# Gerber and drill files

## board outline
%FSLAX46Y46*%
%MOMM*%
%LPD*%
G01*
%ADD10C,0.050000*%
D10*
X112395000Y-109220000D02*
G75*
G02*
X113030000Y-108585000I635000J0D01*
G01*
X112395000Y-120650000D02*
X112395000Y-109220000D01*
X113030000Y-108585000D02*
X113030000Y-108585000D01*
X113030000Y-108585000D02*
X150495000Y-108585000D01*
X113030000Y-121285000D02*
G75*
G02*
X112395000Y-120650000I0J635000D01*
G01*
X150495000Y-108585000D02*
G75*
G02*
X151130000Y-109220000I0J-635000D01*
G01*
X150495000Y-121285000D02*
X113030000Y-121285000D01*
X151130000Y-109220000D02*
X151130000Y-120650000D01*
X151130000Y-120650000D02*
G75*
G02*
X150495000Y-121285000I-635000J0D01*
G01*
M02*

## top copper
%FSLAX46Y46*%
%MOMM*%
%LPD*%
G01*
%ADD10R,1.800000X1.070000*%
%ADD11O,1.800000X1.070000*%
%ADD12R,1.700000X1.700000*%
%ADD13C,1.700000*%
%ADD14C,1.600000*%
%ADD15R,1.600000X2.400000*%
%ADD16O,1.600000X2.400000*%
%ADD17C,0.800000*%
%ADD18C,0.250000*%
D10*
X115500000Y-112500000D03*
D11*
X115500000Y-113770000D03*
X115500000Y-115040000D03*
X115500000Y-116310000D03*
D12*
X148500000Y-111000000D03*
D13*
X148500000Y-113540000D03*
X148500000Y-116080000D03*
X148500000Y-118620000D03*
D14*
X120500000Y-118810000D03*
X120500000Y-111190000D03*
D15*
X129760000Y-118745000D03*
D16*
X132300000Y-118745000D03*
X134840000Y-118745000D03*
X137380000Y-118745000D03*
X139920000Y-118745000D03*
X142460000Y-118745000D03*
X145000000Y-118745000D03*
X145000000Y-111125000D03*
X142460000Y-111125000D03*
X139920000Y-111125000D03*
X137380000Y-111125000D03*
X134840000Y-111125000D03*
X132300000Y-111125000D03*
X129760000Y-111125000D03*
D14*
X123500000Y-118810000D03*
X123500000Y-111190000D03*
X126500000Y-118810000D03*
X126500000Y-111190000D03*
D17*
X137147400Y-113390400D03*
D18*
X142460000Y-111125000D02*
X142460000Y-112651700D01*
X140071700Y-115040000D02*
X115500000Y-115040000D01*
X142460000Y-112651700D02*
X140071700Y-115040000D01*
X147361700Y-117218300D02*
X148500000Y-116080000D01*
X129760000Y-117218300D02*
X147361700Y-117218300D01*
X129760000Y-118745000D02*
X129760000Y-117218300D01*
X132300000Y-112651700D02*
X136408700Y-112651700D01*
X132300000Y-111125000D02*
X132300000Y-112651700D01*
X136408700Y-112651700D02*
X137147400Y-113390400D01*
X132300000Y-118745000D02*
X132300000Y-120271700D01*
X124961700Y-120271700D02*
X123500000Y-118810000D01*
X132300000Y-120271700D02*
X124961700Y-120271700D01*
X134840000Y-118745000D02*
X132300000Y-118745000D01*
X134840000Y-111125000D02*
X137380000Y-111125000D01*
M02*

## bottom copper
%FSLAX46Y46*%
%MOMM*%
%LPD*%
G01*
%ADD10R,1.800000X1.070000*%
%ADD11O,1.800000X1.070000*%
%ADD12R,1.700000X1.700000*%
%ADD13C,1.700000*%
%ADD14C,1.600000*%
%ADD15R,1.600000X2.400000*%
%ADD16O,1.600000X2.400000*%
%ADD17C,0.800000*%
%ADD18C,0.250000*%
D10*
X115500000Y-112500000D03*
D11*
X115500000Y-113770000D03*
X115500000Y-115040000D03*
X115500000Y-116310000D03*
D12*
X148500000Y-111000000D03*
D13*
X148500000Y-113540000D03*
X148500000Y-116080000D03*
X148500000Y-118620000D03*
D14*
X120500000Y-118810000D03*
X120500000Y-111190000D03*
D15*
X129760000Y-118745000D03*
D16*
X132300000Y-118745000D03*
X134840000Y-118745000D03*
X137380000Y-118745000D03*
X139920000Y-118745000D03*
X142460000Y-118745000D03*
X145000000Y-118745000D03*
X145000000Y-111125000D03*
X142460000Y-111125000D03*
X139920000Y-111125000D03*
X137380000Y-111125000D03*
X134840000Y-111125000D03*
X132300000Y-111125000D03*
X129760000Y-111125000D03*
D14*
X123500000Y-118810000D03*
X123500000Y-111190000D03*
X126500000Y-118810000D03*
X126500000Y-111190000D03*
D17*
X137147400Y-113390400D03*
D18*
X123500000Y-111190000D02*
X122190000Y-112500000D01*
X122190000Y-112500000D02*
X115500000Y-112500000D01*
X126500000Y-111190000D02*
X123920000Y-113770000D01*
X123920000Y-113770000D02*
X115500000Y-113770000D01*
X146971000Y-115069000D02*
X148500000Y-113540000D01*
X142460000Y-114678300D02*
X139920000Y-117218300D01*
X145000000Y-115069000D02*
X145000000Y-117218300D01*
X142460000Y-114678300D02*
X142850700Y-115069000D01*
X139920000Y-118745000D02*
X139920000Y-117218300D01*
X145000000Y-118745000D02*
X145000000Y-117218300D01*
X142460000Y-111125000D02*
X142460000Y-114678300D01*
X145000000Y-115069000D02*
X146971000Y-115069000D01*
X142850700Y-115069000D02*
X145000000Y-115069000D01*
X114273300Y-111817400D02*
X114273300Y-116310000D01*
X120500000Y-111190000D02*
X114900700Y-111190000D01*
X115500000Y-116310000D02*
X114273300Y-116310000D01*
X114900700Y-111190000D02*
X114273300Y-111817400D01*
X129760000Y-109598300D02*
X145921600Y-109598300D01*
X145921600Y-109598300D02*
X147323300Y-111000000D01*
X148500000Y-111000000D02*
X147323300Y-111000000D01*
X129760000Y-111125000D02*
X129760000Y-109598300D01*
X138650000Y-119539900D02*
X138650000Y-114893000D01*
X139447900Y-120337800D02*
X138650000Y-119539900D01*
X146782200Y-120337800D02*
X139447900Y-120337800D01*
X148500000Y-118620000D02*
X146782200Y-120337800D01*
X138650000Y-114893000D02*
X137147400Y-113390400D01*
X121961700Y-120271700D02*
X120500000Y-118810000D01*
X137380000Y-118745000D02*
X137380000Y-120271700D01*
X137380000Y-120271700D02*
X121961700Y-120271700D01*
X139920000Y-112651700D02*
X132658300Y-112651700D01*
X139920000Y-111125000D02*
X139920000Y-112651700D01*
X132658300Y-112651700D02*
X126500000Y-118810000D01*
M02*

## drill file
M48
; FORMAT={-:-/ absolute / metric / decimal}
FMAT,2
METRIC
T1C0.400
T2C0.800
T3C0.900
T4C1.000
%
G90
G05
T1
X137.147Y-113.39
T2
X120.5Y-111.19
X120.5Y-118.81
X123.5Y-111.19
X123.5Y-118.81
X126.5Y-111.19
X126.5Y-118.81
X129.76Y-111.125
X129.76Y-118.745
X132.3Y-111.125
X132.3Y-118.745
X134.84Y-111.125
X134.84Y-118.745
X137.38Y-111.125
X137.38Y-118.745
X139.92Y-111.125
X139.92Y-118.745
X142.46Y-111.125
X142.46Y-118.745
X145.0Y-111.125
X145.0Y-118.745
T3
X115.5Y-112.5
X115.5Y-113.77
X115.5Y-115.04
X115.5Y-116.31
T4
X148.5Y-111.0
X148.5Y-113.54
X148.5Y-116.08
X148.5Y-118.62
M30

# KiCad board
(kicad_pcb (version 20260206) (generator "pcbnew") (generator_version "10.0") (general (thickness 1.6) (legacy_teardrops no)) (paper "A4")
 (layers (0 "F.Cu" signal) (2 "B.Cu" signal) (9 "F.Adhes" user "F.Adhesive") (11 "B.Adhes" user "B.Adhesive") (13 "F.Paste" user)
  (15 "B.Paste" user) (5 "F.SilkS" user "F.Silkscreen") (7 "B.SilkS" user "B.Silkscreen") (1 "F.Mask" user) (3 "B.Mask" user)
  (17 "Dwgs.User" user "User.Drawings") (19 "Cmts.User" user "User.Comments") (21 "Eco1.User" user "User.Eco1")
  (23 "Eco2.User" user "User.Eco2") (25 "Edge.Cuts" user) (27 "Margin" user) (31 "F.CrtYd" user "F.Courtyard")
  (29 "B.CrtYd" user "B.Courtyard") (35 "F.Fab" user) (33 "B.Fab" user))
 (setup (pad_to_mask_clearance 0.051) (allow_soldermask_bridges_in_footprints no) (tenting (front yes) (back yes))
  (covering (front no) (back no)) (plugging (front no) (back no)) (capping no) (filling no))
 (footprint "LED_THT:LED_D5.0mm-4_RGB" (layer "F.Cu") (at 115.5 112.5 -90)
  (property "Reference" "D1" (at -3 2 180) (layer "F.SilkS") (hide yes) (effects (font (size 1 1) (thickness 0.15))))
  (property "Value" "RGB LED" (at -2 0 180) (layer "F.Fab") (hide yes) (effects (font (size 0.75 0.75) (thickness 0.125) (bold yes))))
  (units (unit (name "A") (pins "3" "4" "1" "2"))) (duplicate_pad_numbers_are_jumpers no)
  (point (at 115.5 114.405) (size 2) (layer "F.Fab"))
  (pad "1" thru_hole rect (at 0 0 270) (size 1.07 1.8) (drill 0.9) (layers "*.Cu" "*.Mask") (remove_unused_layers no) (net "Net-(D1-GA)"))
  (pad "2" thru_hole oval (at 1.27 0 270) (size 1.07 1.8) (drill 0.9) (layers "*.Cu" "*.Mask") (remove_unused_layers no) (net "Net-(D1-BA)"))
  (pad "3" thru_hole oval (at 2.54 0 270) (size 1.07 1.8) (drill 0.9) (layers "*.Cu" "*.Mask") (remove_unused_layers no) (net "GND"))
  (pad "4" thru_hole oval (at 3.81 0 270) (size 1.07 1.8) (drill 0.9) (layers "*.Cu" "*.Mask") (remove_unused_layers no) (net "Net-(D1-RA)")))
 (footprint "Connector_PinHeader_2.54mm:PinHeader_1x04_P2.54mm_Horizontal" (layer "F.Cu") (at 148.5 111)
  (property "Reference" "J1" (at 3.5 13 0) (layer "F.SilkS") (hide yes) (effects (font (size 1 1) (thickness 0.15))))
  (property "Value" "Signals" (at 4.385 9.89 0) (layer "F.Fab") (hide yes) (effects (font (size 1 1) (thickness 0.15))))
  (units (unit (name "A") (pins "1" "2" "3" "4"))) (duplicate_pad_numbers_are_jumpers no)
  (pad "1" thru_hole rect (at 0 0) (size 1.7 1.7) (drill 1) (layers "*.Cu" "*.Mask") (remove_unused_layers no) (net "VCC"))
  (pad "2" thru_hole circle (at 0 2.54) (size 1.7 1.7) (drill 1) (layers "*.Cu" "*.Mask") (remove_unused_layers no) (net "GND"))
  (pad "3" thru_hole circle (at 0 5.08) (size 1.7 1.7) (drill 1) (layers "*.Cu" "*.Mask") (remove_unused_layers no) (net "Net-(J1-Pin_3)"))
  (pad "4" thru_hole circle (at 0 7.62) (size 1.7 1.7) (drill 1) (layers "*.Cu" "*.Mask") (remove_unused_layers no) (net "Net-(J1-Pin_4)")))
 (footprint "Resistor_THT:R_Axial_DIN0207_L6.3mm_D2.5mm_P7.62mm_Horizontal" (layer "F.Cu") (at 120.5 118.81 90)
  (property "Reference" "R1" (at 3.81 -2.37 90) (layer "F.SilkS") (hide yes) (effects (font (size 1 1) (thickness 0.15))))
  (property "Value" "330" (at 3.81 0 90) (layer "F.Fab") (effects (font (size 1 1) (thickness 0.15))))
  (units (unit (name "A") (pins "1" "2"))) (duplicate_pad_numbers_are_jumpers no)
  (pad "1" thru_hole circle (at 0 0 90) (size 1.6 1.6) (drill 0.8) (layers "*.Cu" "*.Mask") (remove_unused_layers no) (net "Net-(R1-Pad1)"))
  (pad "2" thru_hole circle (at 7.62 0 90) (size 1.6 1.6) (drill 0.8) (layers "*.Cu" "*.Mask") (remove_unused_layers no) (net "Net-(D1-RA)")))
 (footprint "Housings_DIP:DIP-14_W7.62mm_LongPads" (layer "F.Cu") (at 129.76 118.745 90)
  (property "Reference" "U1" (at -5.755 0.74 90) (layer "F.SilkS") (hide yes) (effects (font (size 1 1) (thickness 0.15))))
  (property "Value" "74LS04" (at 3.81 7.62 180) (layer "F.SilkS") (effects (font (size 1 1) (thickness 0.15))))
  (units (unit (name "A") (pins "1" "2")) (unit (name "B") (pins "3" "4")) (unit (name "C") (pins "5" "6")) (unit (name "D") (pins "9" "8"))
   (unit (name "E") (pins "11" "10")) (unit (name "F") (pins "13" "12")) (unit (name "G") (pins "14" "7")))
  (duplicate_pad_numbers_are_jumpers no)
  (pad "1" thru_hole rect (at 0 0 90) (size 2.4 1.6) (drill 0.8) (layers "*.Cu" "*.Mask") (remove_unused_layers no) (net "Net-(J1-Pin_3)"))
  (pad "2" thru_hole oval (at 0 2.54 90) (size 2.4 1.6) (drill 0.8) (layers "*.Cu" "*.Mask") (remove_unused_layers no) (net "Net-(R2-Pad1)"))
  (pad "3" thru_hole oval (at 0 5.08 90) (size 2.4 1.6) (drill 0.8) (layers "*.Cu" "*.Mask") (remove_unused_layers no) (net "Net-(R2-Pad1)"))
  (pad "4" thru_hole oval (at 0 7.62 90) (size 2.4 1.6) (drill 0.8) (layers "*.Cu" "*.Mask") (remove_unused_layers no) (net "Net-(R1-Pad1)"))
  (pad "5" thru_hole oval (at 0 10.16 90) (size 2.4 1.6) (drill 0.8) (layers "*.Cu" "*.Mask") (remove_unused_layers no) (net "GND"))
  (pad "6" thru_hole oval (at 0 12.7 90) (size 2.4 1.6) (drill 0.8) (layers "*.Cu" "*.Mask") (remove_unused_layers no)
   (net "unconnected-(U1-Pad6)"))
  (pad "7" thru_hole oval (at 0 15.24 90) (size 2.4 1.6) (drill 0.8) (layers "*.Cu" "*.Mask") (remove_unused_layers no) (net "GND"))
  (pad "8" thru_hole oval (at 7.62 15.24 90) (size 2.4 1.6) (drill 0.8) (layers "*.Cu" "*.Mask") (remove_unused_layers no)
   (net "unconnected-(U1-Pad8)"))
  (pad "9" thru_hole oval (at 7.62 12.7 90) (size 2.4 1.6) (drill 0.8) (layers "*.Cu" "*.Mask") (remove_unused_layers no) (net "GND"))
  (pad "10" thru_hole oval (at 7.62 10.16 90) (size 2.4 1.6) (drill 0.8) (layers "*.Cu" "*.Mask") (remove_unused_layers no)
   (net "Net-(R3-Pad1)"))
  (pad "11" thru_hole oval (at 7.62 7.62 90) (size 2.4 1.6) (drill 0.8) (layers "*.Cu" "*.Mask") (remove_unused_layers no)
   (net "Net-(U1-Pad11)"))
  (pad "12" thru_hole oval (at 7.62 5.08 90) (size 2.4 1.6) (drill 0.8) (layers "*.Cu" "*.Mask") (remove_unused_layers no)
   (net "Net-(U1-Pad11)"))
  (pad "13" thru_hole oval (at 7.62 2.54 90) (size 2.4 1.6) (drill 0.8) (layers "*.Cu" "*.Mask") (remove_unused_layers no)
   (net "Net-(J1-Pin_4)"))
  (pad "14" thru_hole oval (at 7.62 0 90) (size 2.4 1.6) (drill 0.8) (layers "*.Cu" "*.Mask") (remove_unused_layers no) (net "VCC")))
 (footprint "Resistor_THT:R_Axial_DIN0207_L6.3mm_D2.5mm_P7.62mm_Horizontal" (layer "F.Cu") (at 123.5 118.81 90)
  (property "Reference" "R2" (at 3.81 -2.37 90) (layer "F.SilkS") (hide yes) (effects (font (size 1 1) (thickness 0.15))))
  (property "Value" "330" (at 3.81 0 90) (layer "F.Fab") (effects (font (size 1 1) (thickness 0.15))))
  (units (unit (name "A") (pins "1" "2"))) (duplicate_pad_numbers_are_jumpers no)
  (pad "1" thru_hole circle (at 0 0 90) (size 1.6 1.6) (drill 0.8) (layers "*.Cu" "*.Mask") (remove_unused_layers no) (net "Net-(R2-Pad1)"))
  (pad "2" thru_hole circle (at 7.62 0 90) (size 1.6 1.6) (drill 0.8) (layers "*.Cu" "*.Mask") (remove_unused_layers no) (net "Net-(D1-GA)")))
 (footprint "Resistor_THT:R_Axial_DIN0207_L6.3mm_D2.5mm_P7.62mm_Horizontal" (layer "F.Cu") (at 126.5 118.81 90)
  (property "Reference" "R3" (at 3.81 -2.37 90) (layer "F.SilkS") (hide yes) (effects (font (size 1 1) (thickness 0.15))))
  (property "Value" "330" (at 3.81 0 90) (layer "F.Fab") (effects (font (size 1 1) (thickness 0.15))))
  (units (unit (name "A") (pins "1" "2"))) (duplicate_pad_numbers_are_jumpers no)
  (pad "1" thru_hole circle (at 0 0 90) (size 1.6 1.6) (drill 0.8) (layers "*.Cu" "*.Mask") (remove_unused_layers no) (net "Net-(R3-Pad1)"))
  (pad "2" thru_hole circle (at 7.62 0 90) (size 1.6 1.6) (drill 0.8) (layers "*.Cu" "*.Mask") (remove_unused_layers no) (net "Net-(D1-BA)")))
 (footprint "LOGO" (layer "F.Cu") (at 113.5 119.5)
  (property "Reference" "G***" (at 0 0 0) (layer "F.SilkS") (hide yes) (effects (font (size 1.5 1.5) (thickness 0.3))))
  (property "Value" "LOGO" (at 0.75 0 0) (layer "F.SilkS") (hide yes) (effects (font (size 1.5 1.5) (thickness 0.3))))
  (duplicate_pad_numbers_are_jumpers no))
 (gr_arc (start 112.395 109.22) (mid 112.580987 108.770987) (end 113.03 108.585) (stroke (width 0.05) (type solid)) (layer "Edge.Cuts"))
 (gr_line (start 112.395 120.65) (end 112.395 109.22) (stroke (width 0.05) (type solid)) (layer "Edge.Cuts"))
 (gr_line (start 113.03 108.585) (end 113.03 108.585) (stroke (width 0.05) (type solid)) (layer "Edge.Cuts"))
 (gr_line (start 113.03 108.585) (end 150.495 108.585) (stroke (width 0.05) (type solid)) (layer "Edge.Cuts"))
 (gr_arc (start 113.03 121.285) (mid 112.580987 121.099013) (end 112.395 120.65) (stroke (width 0.05) (type solid)) (layer "Edge.Cuts"))
 (gr_arc (start 150.495 108.585) (mid 150.944013 108.770987) (end 151.13 109.22) (stroke (width 0.05) (type solid)) (layer "Edge.Cuts"))
 (gr_line (start 150.495 121.285) (end 113.03 121.285) (stroke (width 0.05) (type solid)) (layer "Edge.Cuts"))
 (gr_line (start 151.13 109.22) (end 151.13 120.65) (stroke (width 0.05) (type solid)) (layer "Edge.Cuts"))
 (gr_arc (start 151.13 120.65) (mid 150.944013 121.099013) (end 150.495 121.285) (stroke (width 0.05) (type solid)) (layer "Edge.Cuts"))
 (segment (start 123.5 111.19) (end 122.19 112.5) (width 0.25) (layer "B.Cu") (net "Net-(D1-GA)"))
 (segment (start 122.19 112.5) (end 115.5 112.5) (width 0.25) (layer "B.Cu") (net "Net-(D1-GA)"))
 (segment (start 126.5 111.19) (end 123.92 113.77) (width 0.25) (layer "B.Cu") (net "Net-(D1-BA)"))
 (segment (start 123.92 113.77) (end 115.5 113.77) (width 0.25) (layer "B.Cu") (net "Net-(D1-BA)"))
 (segment (start 142.46 111.125) (end 142.46 112.6517) (width 0.25) (layer "F.Cu") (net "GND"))
 (segment (start 140.0717 115.04) (end 115.5 115.04) (width 0.25) (layer "F.Cu") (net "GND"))
 (segment (start 142.46 112.6517) (end 140.0717 115.04) (width 0.25) (layer "F.Cu") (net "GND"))
 (segment (start 146.971 115.069) (end 148.5 113.54) (width 0.25) (layer "B.Cu") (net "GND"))
 (segment (start 142.46 114.6783) (end 139.92 117.2183) (width 0.25) (layer "B.Cu") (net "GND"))
 (segment (start 145 115.069) (end 145 117.2183) (width 0.25) (layer "B.Cu") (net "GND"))
 (segment (start 142.46 114.6783) (end 142.8507 115.069) (width 0.25) (layer "B.Cu") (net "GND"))
 (segment (start 139.92 118.745) (end 139.92 117.2183) (width 0.25) (layer "B.Cu") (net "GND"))
 (segment (start 145 118.745) (end 145 117.2183) (width 0.25) (layer "B.Cu") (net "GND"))
 (segment (start 142.46 111.125) (end 142.46 114.6783) (width 0.25) (layer "B.Cu") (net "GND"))
 (segment (start 145 115.069) (end 146.971 115.069) (width 0.25) (layer "B.Cu") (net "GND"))
 (segment (start 142.8507 115.069) (end 145 115.069) (width 0.25) (layer "B.Cu") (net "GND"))
 (segment (start 114.2733 111.8174) (end 114.2733 116.31) (width 0.25) (layer "B.Cu") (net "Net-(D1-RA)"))
 (segment (start 120.5 111.19) (end 114.9007 111.19) (width 0.25) (layer "B.Cu") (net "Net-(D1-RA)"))
 (segment (start 115.5 116.31) (end 114.2733 116.31) (width 0.25) (layer "B.Cu") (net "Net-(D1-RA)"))
 (segment (start 114.9007 111.19) (end 114.2733 111.8174) (width 0.25) (layer "B.Cu") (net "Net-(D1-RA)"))
 (segment (start 129.76 109.5983) (end 145.9216 109.5983) (width 0.25) (layer "B.Cu") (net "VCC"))
 (segment (start 145.9216 109.5983) (end 147.3233 111) (width 0.25) (layer "B.Cu") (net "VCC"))
 (segment (start 148.5 111) (end 147.3233 111) (width 0.25) (layer "B.Cu") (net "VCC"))
 (segment (start 129.76 111.125) (end 129.76 109.5983) (width 0.25) (layer "B.Cu") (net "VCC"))
 (segment (start 147.3617 117.2183) (end 148.5 116.08) (width 0.25) (layer "F.Cu") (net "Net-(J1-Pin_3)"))
 (segment (start 129.76 117.2183) (end 147.3617 117.2183) (width 0.25) (layer "F.Cu") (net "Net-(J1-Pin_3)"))
 (segment (start 129.76 118.745) (end 129.76 117.2183) (width 0.25) (layer "F.Cu") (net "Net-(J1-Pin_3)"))
 (segment (start 132.3 112.6517) (end 136.4087 112.6517) (width 0.25) (layer "F.Cu") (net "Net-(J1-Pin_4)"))
 (segment (start 132.3 111.125) (end 132.3 112.6517) (width 0.25) (layer "F.Cu") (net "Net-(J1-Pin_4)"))
 (segment (start 136.4087 112.6517) (end 137.1474 113.3904) (width 0.25) (layer "F.Cu") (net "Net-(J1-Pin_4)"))
 (via (at 137.1474 113.3904) (size 0.8) (drill 0.4) (layers "F.Cu" "B.Cu") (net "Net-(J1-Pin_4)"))
 (segment (start 138.65 119.5399) (end 138.65 114.893) (width 0.25) (layer "B.Cu") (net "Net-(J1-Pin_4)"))
 (segment (start 139.4479 120.3378) (end 138.65 119.5399) (width 0.25) (layer "B.Cu") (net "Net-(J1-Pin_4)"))
 (segment (start 146.7822 120.3378) (end 139.4479 120.3378) (width 0.25) (layer "B.Cu") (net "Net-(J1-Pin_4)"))
 (segment (start 148.5 118.62) (end 146.7822 120.3378) (width 0.25) (layer "B.Cu") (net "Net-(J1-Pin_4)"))
 (segment (start 138.65 114.893) (end 137.1474 113.3904) (width 0.25) (layer "B.Cu") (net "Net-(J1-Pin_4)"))
 (segment (start 121.9617 120.2717) (end 120.5 118.81) (width 0.25) (layer "B.Cu") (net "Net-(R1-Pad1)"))
 (segment (start 137.38 118.745) (end 137.38 120.2717) (width 0.25) (layer "B.Cu") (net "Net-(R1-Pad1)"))
 (segment (start 137.38 120.2717) (end 121.9617 120.2717) (width 0.25) (layer "B.Cu") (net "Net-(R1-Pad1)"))
 (segment (start 132.3 118.745) (end 132.3 120.2717) (width 0.25) (layer "F.Cu") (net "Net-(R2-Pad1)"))
 (segment (start 124.9617 120.2717) (end 123.5 118.81) (width 0.25) (layer "F.Cu") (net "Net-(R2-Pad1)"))
 (segment (start 132.3 120.2717) (end 124.9617 120.2717) (width 0.25) (layer "F.Cu") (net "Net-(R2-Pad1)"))
 (segment (start 134.84 118.745) (end 132.3 118.745) (width 0.25) (layer "F.Cu") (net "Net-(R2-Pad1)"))
 (segment (start 139.92 112.6517) (end 132.6583 112.6517) (width 0.25) (layer "B.Cu") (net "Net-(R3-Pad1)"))
 (segment (start 139.92 111.125) (end 139.92 112.6517) (width 0.25) (layer "B.Cu") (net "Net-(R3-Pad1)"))
 (segment (start 132.6583 112.6517) (end 126.5 118.81) (width 0.25) (layer "B.Cu") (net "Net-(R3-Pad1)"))
 (segment (start 134.84 111.125) (end 137.38 111.125) (width 0.25) (layer "F.Cu") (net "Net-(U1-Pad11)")))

